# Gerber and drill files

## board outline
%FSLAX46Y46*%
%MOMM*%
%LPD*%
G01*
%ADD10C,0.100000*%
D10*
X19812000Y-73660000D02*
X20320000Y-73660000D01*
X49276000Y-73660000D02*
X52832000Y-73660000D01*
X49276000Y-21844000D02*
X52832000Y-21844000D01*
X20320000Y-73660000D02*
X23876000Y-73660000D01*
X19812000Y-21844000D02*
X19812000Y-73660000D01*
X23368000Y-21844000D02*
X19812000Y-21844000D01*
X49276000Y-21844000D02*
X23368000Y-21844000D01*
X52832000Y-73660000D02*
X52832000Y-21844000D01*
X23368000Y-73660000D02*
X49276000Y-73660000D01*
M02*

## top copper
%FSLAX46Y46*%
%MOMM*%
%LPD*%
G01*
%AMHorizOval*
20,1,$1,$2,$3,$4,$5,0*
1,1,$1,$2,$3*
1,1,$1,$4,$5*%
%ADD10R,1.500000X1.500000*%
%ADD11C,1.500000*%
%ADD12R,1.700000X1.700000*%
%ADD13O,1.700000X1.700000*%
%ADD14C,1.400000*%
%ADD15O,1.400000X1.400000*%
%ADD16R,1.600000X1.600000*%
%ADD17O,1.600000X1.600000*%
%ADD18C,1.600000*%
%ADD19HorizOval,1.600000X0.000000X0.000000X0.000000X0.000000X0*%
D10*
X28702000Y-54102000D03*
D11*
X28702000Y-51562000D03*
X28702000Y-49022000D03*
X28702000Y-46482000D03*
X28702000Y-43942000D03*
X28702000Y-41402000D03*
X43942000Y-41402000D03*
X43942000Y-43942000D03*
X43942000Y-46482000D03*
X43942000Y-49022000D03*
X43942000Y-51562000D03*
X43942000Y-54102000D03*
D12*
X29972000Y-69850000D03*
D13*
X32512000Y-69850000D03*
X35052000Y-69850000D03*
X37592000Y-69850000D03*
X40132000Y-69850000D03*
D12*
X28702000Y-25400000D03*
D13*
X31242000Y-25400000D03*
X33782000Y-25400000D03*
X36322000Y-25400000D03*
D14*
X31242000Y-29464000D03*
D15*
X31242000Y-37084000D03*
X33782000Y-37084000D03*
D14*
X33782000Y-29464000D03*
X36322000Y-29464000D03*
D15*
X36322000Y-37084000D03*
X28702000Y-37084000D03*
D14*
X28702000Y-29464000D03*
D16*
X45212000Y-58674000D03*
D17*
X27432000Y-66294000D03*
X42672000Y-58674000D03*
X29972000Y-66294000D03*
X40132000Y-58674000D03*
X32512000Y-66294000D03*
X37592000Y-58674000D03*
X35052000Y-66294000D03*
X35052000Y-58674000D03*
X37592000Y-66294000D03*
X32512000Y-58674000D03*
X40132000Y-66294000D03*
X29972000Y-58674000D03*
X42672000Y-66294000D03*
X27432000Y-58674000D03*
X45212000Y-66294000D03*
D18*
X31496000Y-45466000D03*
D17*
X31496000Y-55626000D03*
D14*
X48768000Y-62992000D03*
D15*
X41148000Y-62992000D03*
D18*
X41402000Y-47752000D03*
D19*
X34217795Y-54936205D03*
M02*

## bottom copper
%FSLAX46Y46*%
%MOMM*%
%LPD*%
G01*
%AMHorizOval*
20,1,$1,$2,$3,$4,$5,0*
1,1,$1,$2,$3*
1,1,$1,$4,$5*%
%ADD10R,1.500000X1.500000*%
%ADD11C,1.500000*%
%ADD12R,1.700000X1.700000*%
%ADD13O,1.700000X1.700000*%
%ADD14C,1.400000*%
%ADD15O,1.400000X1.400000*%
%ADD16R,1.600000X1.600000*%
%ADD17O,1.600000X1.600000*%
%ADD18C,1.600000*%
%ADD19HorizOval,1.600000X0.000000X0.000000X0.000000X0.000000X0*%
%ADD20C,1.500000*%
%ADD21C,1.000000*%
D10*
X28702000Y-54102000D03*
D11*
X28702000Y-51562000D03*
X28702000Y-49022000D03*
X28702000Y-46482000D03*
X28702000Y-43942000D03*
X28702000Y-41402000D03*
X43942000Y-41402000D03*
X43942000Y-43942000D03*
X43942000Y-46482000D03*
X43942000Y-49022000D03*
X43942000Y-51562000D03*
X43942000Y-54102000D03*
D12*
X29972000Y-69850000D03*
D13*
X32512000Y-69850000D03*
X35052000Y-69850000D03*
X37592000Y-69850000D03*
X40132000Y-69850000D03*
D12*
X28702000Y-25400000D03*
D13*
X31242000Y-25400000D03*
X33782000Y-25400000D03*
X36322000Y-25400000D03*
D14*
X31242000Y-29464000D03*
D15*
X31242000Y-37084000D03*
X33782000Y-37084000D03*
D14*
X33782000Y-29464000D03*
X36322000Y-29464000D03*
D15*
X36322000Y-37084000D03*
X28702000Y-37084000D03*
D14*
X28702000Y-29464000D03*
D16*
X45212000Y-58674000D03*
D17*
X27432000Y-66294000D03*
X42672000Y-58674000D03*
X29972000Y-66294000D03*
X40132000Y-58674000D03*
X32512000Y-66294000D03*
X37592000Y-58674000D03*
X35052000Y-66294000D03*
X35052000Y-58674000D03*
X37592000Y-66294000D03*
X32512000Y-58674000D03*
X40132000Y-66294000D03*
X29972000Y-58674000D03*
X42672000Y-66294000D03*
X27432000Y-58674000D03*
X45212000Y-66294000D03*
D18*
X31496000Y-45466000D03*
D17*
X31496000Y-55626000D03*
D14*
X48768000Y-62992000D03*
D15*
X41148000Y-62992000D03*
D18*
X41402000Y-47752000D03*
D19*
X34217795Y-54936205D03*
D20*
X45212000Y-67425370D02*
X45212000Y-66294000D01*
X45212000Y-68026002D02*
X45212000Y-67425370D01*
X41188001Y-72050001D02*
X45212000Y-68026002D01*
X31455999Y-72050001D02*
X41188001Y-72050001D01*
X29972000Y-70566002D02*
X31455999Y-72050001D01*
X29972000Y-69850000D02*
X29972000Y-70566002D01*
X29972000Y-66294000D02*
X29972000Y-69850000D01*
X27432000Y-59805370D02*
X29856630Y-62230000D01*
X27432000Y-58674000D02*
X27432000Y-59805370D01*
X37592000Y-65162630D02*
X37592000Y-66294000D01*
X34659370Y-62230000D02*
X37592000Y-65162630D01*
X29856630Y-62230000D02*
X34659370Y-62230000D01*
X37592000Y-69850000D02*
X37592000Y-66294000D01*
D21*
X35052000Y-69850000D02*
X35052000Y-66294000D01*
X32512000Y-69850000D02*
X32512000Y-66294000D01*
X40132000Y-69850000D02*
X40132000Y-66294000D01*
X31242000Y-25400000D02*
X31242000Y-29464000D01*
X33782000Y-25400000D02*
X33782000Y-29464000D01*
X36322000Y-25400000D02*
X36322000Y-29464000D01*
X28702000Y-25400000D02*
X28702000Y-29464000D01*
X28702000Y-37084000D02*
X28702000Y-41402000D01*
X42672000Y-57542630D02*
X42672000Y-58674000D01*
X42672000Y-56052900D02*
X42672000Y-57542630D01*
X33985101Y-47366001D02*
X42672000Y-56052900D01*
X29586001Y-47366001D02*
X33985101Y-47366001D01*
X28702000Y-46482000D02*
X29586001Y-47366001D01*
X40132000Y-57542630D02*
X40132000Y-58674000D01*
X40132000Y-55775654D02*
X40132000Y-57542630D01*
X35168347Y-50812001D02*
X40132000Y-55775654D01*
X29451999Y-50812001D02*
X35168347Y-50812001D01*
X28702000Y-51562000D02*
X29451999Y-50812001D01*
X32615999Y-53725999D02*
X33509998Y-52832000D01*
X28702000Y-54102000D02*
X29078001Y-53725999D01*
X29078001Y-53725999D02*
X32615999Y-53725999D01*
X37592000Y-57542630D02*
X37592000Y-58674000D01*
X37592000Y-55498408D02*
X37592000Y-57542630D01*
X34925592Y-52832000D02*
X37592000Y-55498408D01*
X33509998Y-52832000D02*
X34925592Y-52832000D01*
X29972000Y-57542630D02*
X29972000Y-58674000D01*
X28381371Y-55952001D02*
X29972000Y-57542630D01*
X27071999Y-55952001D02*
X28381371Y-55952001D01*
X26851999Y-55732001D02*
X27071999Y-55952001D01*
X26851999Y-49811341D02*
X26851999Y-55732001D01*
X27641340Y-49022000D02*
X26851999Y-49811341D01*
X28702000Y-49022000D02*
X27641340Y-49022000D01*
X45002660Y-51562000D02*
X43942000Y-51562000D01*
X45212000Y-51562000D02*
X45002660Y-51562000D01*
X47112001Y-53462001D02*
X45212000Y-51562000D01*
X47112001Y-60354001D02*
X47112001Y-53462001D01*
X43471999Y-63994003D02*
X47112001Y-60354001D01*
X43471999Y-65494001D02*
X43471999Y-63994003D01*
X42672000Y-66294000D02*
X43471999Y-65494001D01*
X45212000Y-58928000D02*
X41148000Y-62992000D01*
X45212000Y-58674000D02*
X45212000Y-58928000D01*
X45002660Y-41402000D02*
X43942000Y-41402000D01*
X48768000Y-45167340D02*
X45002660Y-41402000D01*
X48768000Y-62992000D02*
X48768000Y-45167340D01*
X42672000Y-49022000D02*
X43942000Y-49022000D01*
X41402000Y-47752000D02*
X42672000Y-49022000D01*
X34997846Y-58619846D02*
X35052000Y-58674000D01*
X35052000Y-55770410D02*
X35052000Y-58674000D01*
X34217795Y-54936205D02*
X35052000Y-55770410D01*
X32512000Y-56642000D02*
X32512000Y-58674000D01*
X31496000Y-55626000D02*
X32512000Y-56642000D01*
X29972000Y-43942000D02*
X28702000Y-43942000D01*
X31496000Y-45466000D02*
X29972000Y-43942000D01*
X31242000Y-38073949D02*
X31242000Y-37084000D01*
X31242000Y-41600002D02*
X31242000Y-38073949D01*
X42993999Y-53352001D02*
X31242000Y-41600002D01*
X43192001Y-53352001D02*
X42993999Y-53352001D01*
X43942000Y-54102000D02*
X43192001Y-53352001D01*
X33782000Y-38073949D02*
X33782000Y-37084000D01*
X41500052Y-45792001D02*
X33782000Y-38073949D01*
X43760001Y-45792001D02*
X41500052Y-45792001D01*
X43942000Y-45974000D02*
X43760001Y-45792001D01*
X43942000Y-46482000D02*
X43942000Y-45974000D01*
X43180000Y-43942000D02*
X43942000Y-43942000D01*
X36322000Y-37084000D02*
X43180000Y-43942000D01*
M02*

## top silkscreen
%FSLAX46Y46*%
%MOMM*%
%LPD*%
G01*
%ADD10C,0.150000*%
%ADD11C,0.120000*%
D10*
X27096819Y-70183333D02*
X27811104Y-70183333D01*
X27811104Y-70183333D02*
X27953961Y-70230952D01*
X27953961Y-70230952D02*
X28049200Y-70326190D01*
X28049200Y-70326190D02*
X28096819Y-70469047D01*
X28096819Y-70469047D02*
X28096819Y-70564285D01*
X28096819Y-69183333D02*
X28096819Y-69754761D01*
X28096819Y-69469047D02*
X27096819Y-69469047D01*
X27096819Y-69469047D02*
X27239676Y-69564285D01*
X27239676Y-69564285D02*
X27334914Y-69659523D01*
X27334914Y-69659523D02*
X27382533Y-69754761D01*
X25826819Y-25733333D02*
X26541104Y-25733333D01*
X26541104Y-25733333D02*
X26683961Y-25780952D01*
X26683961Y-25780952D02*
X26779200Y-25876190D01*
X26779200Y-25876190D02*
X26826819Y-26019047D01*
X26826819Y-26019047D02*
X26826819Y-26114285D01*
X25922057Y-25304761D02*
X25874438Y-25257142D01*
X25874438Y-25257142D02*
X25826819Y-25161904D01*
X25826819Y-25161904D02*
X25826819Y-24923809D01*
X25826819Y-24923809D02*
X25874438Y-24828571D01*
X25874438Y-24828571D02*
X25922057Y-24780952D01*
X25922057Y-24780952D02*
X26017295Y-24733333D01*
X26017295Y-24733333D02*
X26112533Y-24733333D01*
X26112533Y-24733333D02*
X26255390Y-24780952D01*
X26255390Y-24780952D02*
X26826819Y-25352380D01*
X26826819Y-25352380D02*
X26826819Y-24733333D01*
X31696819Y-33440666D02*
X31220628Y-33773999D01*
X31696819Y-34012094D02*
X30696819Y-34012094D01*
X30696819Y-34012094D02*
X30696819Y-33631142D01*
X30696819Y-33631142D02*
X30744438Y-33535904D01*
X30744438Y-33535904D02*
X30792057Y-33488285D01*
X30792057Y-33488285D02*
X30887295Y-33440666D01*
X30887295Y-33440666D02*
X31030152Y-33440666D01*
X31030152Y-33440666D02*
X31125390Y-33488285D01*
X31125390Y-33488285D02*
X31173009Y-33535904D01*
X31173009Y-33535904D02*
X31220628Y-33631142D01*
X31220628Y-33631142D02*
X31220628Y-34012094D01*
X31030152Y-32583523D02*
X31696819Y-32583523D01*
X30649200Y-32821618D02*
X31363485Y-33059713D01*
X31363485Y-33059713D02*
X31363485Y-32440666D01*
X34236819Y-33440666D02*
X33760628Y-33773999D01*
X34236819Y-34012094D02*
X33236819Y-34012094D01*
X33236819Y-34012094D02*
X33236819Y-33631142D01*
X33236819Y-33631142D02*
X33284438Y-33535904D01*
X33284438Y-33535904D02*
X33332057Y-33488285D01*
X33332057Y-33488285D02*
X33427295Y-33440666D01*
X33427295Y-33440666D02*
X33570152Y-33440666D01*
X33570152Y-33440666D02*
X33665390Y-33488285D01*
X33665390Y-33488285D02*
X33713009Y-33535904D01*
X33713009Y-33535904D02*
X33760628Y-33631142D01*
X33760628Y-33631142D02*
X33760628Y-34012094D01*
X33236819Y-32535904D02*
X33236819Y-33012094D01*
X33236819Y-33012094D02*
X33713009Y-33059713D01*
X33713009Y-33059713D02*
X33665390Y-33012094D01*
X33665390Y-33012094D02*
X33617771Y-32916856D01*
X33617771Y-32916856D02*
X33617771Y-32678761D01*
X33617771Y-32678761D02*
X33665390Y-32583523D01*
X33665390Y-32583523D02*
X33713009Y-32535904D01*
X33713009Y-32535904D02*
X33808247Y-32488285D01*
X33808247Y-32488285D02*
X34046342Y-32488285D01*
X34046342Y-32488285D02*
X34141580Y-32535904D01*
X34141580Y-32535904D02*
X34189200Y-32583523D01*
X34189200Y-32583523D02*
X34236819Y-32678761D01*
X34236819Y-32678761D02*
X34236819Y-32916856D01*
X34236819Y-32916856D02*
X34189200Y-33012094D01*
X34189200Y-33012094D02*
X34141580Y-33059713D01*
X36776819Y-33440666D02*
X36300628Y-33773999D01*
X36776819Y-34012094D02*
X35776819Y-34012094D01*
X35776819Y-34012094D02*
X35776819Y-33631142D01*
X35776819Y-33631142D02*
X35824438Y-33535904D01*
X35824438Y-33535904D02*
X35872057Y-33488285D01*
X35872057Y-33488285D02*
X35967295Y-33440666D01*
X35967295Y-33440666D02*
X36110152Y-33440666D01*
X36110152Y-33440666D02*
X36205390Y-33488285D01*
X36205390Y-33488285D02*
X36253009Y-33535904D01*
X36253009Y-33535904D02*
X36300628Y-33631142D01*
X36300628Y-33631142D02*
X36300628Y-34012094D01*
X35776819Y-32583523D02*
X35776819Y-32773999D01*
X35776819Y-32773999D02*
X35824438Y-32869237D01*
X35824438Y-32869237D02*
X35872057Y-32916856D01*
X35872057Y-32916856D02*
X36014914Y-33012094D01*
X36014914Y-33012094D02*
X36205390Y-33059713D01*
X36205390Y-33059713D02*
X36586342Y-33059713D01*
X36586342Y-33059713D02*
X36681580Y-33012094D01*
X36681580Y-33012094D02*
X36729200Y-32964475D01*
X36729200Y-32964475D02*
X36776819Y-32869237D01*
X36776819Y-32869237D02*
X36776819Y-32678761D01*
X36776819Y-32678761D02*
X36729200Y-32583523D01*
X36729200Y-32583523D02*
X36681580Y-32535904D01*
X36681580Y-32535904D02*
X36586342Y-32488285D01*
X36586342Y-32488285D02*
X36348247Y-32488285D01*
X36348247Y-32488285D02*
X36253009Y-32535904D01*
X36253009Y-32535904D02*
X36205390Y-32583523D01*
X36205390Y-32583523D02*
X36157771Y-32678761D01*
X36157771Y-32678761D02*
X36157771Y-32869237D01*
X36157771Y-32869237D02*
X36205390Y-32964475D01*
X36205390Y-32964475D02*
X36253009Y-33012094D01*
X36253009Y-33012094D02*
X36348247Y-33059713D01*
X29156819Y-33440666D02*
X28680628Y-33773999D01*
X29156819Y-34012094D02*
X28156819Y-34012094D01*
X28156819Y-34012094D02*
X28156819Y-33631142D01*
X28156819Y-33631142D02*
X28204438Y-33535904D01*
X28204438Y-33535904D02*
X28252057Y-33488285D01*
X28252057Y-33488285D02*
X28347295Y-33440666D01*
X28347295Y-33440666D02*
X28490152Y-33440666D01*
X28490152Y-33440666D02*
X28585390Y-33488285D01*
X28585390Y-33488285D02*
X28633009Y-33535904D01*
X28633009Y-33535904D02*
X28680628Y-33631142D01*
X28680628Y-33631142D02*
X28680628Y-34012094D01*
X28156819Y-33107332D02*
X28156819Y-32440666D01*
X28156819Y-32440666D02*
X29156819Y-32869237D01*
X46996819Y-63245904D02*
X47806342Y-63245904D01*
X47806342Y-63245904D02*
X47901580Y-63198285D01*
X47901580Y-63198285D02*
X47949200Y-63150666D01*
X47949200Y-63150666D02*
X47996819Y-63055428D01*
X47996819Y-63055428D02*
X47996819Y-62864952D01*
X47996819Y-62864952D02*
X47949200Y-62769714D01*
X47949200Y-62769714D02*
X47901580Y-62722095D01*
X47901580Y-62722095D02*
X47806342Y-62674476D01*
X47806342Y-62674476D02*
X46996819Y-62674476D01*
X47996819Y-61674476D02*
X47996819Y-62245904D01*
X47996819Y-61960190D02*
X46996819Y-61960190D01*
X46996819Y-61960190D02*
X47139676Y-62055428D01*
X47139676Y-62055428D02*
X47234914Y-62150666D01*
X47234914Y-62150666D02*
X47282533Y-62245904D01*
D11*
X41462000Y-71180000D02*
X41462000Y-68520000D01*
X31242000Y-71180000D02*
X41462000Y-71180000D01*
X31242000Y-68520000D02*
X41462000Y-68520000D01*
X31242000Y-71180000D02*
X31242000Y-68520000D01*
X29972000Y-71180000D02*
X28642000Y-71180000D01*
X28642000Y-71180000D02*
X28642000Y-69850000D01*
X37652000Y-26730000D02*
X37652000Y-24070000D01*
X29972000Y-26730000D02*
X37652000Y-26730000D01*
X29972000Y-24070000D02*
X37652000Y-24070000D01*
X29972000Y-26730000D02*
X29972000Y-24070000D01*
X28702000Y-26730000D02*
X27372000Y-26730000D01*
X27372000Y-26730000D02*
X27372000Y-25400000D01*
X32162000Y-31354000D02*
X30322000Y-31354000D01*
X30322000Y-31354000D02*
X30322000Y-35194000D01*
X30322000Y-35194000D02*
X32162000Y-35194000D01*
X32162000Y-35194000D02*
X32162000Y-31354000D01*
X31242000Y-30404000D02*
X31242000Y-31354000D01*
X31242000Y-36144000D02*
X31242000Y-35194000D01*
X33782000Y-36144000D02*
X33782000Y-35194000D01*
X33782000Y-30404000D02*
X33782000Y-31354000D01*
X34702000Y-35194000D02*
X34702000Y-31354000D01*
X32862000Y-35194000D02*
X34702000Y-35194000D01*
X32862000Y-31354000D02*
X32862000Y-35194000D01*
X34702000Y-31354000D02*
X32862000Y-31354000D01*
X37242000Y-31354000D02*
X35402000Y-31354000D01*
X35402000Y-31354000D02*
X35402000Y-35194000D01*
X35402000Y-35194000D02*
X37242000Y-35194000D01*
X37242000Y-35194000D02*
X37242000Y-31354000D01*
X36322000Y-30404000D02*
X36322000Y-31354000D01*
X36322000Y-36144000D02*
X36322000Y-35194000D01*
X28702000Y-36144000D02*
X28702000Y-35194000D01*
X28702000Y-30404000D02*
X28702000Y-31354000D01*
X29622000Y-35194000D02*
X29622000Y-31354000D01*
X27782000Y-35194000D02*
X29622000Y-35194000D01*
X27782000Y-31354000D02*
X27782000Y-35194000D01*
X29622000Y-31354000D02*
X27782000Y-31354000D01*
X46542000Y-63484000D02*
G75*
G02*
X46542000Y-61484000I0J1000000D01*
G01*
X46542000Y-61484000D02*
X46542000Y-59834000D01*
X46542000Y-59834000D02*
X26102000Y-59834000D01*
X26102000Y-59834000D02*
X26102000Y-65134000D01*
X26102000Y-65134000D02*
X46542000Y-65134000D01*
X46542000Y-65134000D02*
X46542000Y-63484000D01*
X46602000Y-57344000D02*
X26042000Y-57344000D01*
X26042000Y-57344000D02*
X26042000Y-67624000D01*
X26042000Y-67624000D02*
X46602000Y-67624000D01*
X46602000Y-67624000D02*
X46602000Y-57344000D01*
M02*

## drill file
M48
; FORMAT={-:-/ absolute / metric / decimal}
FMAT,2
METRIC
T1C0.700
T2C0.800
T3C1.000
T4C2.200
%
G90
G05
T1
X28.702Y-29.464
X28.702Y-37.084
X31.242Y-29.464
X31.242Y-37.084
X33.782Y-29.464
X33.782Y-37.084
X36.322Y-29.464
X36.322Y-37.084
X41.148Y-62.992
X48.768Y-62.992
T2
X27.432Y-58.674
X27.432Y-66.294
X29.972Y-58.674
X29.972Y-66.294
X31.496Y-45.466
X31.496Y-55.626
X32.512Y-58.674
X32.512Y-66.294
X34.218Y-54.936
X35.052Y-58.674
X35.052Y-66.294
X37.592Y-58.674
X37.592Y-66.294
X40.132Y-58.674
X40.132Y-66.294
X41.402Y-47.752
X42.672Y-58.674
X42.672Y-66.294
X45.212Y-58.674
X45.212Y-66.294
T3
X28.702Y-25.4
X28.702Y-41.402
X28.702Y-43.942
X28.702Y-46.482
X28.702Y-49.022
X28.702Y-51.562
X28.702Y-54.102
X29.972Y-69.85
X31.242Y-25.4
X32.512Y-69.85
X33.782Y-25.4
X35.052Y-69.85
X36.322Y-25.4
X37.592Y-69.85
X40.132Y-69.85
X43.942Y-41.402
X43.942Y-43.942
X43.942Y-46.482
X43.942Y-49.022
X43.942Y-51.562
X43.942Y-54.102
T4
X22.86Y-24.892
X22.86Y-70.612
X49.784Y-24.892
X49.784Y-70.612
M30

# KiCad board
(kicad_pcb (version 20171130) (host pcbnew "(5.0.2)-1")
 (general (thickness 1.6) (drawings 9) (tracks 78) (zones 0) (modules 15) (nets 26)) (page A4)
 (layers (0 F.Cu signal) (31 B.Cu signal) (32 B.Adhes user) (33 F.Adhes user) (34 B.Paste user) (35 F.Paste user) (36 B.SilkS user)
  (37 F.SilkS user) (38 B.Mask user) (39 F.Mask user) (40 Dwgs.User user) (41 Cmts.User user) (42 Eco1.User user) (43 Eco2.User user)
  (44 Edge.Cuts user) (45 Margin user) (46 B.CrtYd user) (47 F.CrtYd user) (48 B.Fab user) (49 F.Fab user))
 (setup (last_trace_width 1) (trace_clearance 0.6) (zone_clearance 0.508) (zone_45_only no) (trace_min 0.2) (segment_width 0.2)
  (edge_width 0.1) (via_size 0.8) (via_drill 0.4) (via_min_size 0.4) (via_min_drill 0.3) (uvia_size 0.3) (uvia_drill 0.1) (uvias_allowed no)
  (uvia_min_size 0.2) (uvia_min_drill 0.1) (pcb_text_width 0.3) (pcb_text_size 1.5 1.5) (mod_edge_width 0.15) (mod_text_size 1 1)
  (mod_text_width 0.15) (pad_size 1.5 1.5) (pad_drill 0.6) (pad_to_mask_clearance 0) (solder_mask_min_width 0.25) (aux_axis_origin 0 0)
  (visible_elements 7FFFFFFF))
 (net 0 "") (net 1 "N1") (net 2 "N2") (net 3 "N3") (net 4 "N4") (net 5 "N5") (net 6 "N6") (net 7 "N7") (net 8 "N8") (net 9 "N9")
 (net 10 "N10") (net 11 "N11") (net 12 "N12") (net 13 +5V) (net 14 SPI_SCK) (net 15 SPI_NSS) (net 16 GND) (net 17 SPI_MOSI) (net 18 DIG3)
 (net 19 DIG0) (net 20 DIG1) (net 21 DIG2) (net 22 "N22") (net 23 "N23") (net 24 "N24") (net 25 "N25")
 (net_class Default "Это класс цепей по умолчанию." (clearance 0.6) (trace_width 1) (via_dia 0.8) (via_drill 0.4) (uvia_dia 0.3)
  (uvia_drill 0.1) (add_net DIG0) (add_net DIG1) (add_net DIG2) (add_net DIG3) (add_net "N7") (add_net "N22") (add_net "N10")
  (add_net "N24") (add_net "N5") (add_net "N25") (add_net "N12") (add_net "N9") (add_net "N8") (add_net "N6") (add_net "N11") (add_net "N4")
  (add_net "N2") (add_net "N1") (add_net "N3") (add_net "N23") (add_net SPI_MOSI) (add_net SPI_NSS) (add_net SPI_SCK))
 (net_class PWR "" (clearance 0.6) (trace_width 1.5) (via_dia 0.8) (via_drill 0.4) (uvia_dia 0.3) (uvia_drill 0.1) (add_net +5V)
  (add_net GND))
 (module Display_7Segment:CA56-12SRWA (layer B.Cu) (at 28.702 54.102)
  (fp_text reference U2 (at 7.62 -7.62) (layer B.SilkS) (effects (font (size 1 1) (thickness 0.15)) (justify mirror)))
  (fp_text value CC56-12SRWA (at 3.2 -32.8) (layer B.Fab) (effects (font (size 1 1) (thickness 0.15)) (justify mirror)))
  (pad 1 thru_hole rect (at 0 0) (size 1.5 1.5) (drill 1) (layers *.Cu *.Mask) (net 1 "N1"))
  (pad 2 thru_hole circle (at 0 -2.54) (size 1.5 1.5) (drill 1) (layers *.Cu *.Mask) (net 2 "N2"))
  (pad 3 thru_hole circle (at 0 -5.08) (size 1.5 1.5) (drill 1) (layers *.Cu *.Mask) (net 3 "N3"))
  (pad 4 thru_hole circle (at 0 -7.62) (size 1.5 1.5) (drill 1) (layers *.Cu *.Mask) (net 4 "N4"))
  (pad 5 thru_hole circle (at 0 -10.16) (size 1.5 1.5) (drill 1) (layers *.Cu *.Mask) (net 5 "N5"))
  (pad 6 thru_hole circle (at 0 -12.7) (size 1.5 1.5) (drill 1) (layers *.Cu *.Mask) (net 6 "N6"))
  (pad 7 thru_hole circle (at 15.24 -12.7) (size 1.5 1.5) (drill 1) (layers *.Cu *.Mask) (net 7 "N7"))
  (pad 8 thru_hole circle (at 15.24 -10.16) (size 1.5 1.5) (drill 1) (layers *.Cu *.Mask) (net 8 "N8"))
  (pad 9 thru_hole circle (at 15.24 -7.62) (size 1.5 1.5) (drill 1) (layers *.Cu *.Mask) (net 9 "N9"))
  (pad 10 thru_hole circle (at 15.24 -5.08) (size 1.5 1.5) (drill 1) (layers *.Cu *.Mask) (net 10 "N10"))
  (pad 11 thru_hole circle (at 15.24 -2.54) (size 1.5 1.5) (drill 1) (layers *.Cu *.Mask) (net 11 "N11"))
  (pad 12 thru_hole circle (at 15.24 0) (size 1.5 1.5) (drill 1) (layers *.Cu *.Mask) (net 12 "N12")))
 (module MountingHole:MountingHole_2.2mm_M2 (layer F.Cu) (at 22.86 24.892)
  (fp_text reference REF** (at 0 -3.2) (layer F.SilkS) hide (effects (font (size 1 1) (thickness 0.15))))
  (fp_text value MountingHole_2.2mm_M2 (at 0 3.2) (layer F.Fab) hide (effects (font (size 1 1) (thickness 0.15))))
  (pad 1 np_thru_hole circle (at 0 0) (size 2.2 2.2) (drill 2.2) (layers *.Cu *.Mask)))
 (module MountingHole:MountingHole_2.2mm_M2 (layer F.Cu) (at 22.86 70.612)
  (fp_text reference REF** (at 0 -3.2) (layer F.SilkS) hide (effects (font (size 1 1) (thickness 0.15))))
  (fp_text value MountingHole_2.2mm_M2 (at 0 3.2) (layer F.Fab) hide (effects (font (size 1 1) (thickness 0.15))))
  (pad 1 np_thru_hole circle (at 0 0) (size 2.2 2.2) (drill 2.2) (layers *.Cu *.Mask)))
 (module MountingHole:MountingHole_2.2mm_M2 (layer F.Cu) (at 49.784 24.892)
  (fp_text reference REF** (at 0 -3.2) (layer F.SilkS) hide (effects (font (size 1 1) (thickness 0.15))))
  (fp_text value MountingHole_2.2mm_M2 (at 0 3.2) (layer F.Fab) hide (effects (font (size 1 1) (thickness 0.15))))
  (pad 1 np_thru_hole circle (at 0 0) (size 2.2 2.2) (drill 2.2) (layers *.Cu *.Mask)))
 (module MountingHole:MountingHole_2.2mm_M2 (layer F.Cu) (at 49.784 70.612)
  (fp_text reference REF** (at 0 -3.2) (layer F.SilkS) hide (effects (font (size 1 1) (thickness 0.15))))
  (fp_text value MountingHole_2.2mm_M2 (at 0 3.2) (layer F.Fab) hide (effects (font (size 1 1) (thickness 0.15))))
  (pad 1 np_thru_hole circle (at 0 0) (size 2.2 2.2) (drill 2.2) (layers *.Cu *.Mask)))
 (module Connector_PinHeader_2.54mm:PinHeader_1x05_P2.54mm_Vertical (layer F.Cu) (at 29.972 69.85 90)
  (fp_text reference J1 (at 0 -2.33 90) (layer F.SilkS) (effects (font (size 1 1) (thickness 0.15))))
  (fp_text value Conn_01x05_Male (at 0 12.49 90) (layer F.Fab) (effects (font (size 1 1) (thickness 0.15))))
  (fp_line (start -1.33 11.49) (end 1.33 11.49) (layer F.SilkS) (width 0.12))
  (fp_line (start -1.33 1.27) (end -1.33 11.49) (layer F.SilkS) (width 0.12))
  (fp_line (start 1.33 1.27) (end 1.33 11.49) (layer F.SilkS) (width 0.12))
  (fp_line (start -1.33 1.27) (end 1.33 1.27) (layer F.SilkS) (width 0.12))
  (fp_line (start -1.33 0) (end -1.33 -1.33) (layer F.SilkS) (width 0.12))
  (fp_line (start -1.33 -1.33) (end 0 -1.33) (layer F.SilkS) (width 0.12))
  (pad 1 thru_hole rect (at 0 0 90) (size 1.7 1.7) (drill 1) (layers *.Cu *.Mask) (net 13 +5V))
  (pad 2 thru_hole oval (at 0 2.54 90) (size 1.7 1.7) (drill 1) (layers *.Cu *.Mask) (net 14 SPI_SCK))
  (pad 3 thru_hole oval (at 0 5.08 90) (size 1.7 1.7) (drill 1) (layers *.Cu *.Mask) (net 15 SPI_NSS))
  (pad 4 thru_hole oval (at 0 7.62 90) (size 1.7 1.7) (drill 1) (layers *.Cu *.Mask) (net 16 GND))
  (pad 5 thru_hole oval (at 0 10.16 90) (size 1.7 1.7) (drill 1) (layers *.Cu *.Mask) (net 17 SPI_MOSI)))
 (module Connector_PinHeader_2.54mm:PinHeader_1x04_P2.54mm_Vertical (layer F.Cu) (at 28.702 25.4 90)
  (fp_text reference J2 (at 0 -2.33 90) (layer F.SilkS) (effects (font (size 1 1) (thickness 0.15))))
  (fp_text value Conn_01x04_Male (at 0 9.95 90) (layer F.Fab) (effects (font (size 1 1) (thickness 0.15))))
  (fp_line (start -1.33 8.95) (end 1.33 8.95) (layer F.SilkS) (width 0.12))
  (fp_line (start -1.33 1.27) (end -1.33 8.95) (layer F.SilkS) (width 0.12))
  (fp_line (start 1.33 1.27) (end 1.33 8.95) (layer F.SilkS) (width 0.12))
  (fp_line (start -1.33 1.27) (end 1.33 1.27) (layer F.SilkS) (width 0.12))
  (fp_line (start -1.33 0) (end -1.33 -1.33) (layer F.SilkS) (width 0.12))
  (fp_line (start -1.33 -1.33) (end 0 -1.33) (layer F.SilkS) (width 0.12))
  (pad 1 thru_hole rect (at 0 0 90) (size 1.7 1.7) (drill 1) (layers *.Cu *.Mask) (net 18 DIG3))
  (pad 2 thru_hole oval (at 0 2.54 90) (size 1.7 1.7) (drill 1) (layers *.Cu *.Mask) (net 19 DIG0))
  (pad 3 thru_hole oval (at 0 5.08 90) (size 1.7 1.7) (drill 1) (layers *.Cu *.Mask) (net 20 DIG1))
  (pad 4 thru_hole oval (at 0 7.62 90) (size 1.7 1.7) (drill 1) (layers *.Cu *.Mask) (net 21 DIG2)))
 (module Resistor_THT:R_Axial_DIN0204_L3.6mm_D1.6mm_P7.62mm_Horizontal (layer F.Cu) (at 31.242 29.464 270)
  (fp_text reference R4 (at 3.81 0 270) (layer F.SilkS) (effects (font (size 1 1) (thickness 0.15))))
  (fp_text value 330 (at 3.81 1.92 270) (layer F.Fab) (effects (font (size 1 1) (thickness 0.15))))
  (fp_line (start 1.89 -0.92) (end 1.89 0.92) (layer F.SilkS) (width 0.12))
  (fp_line (start 1.89 0.92) (end 5.73 0.92) (layer F.SilkS) (width 0.12))
  (fp_line (start 5.73 0.92) (end 5.73 -0.92) (layer F.SilkS) (width 0.12))
  (fp_line (start 5.73 -0.92) (end 1.89 -0.92) (layer F.SilkS) (width 0.12))
  (fp_line (start 0.94 0) (end 1.89 0) (layer F.SilkS) (width 0.12))
  (fp_line (start 6.68 0) (end 5.73 0) (layer F.SilkS) (width 0.12))
  (pad 1 thru_hole circle (at 0 0 270) (size 1.4 1.4) (drill 0.7) (layers *.Cu *.Mask) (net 19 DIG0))
  (pad 2 thru_hole oval (at 7.62 0 270) (size 1.4 1.4) (drill 0.7) (layers *.Cu *.Mask) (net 12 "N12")))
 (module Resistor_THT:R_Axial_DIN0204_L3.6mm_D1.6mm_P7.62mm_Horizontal (layer F.Cu) (at 33.782 29.464 270)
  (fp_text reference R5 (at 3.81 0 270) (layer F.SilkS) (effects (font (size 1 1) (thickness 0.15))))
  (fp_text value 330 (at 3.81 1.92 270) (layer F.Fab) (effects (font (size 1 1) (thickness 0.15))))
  (fp_line (start 6.68 0) (end 5.73 0) (layer F.SilkS) (width 0.12))
  (fp_line (start 0.94 0) (end 1.89 0) (layer F.SilkS) (width 0.12))
  (fp_line (start 5.73 -0.92) (end 1.89 -0.92) (layer F.SilkS) (width 0.12))
  (fp_line (start 5.73 0.92) (end 5.73 -0.92) (layer F.SilkS) (width 0.12))
  (fp_line (start 1.89 0.92) (end 5.73 0.92) (layer F.SilkS) (width 0.12))
  (fp_line (start 1.89 -0.92) (end 1.89 0.92) (layer F.SilkS) (width 0.12))
  (pad 2 thru_hole oval (at 7.62 0 270) (size 1.4 1.4) (drill 0.7) (layers *.Cu *.Mask) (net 9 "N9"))
  (pad 1 thru_hole circle (at 0 0 270) (size 1.4 1.4) (drill 0.7) (layers *.Cu *.Mask) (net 20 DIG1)))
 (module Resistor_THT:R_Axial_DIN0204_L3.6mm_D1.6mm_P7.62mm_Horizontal (layer F.Cu) (at 36.322 29.464 270)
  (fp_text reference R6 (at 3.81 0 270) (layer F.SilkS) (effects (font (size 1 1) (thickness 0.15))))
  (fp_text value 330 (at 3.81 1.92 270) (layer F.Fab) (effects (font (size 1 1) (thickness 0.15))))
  (fp_line (start 1.89 -0.92) (end 1.89 0.92) (layer F.SilkS) (width 0.12))
  (fp_line (start 1.89 0.92) (end 5.73 0.92) (layer F.SilkS) (width 0.12))
  (fp_line (start 5.73 0.92) (end 5.73 -0.92) (layer F.SilkS) (width 0.12))
  (fp_line (start 5.73 -0.92) (end 1.89 -0.92) (layer F.SilkS) (width 0.12))
  (fp_line (start 0.94 0) (end 1.89 0) (layer F.SilkS) (width 0.12))
  (fp_line (start 6.68 0) (end 5.73 0) (layer F.SilkS) (width 0.12))
  (pad 1 thru_hole circle (at 0 0 270) (size 1.4 1.4) (drill 0.7) (layers *.Cu *.Mask) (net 21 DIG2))
  (pad 2 thru_hole oval (at 7.62 0 270) (size 1.4 1.4) (drill 0.7) (layers *.Cu *.Mask) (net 8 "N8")))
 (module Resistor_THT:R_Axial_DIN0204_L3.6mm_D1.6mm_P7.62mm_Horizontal (layer F.Cu) (at 28.702 29.464 270)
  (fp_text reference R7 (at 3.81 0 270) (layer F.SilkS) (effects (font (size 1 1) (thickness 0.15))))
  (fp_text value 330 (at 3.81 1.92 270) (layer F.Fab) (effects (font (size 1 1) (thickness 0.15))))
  (fp_line (start 6.68 0) (end 5.73 0) (layer F.SilkS) (width 0.12))
  (fp_line (start 0.94 0) (end 1.89 0) (layer F.SilkS) (width 0.12))
  (fp_line (start 5.73 -0.92) (end 1.89 -0.92) (layer F.SilkS) (width 0.12))
  (fp_line (start 5.73 0.92) (end 5.73 -0.92) (layer F.SilkS) (width 0.12))
  (fp_line (start 1.89 0.92) (end 5.73 0.92) (layer F.SilkS) (width 0.12))
  (fp_line (start 1.89 -0.92) (end 1.89 0.92) (layer F.SilkS) (width 0.12))
  (pad 2 thru_hole oval (at 7.62 0 270) (size 1.4 1.4) (drill 0.7) (layers *.Cu *.Mask) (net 6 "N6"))
  (pad 1 thru_hole circle (at 0 0 270) (size 1.4 1.4) (drill 0.7) (layers *.Cu *.Mask) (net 18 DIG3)))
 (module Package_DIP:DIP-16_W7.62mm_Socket (layer F.Cu) (at 45.212 58.674 270)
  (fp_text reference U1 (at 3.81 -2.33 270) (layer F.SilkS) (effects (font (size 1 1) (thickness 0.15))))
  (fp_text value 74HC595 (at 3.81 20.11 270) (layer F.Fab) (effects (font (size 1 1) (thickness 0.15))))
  (fp_arc (start 3.81 -1.33) (end 2.81 -1.33) (angle -180) (layer F.SilkS) (width 0.12))
  (fp_line (start 2.81 -1.33) (end 1.16 -1.33) (layer F.SilkS) (width 0.12))
  (fp_line (start 1.16 -1.33) (end 1.16 19.11) (layer F.SilkS) (width 0.12))
  (fp_line (start 1.16 19.11) (end 6.46 19.11) (layer F.SilkS) (width 0.12))
  (fp_line (start 6.46 19.11) (end 6.46 -1.33) (layer F.SilkS) (width 0.12))
  (fp_line (start 6.46 -1.33) (end 4.81 -1.33) (layer F.SilkS) (width 0.12))
  (fp_line (start -1.33 -1.39) (end -1.33 19.17) (layer F.SilkS) (width 0.12))
  (fp_line (start -1.33 19.17) (end 8.95 19.17) (layer F.SilkS) (width 0.12))
  (fp_line (start 8.95 19.17) (end 8.95 -1.39) (layer F.SilkS) (width 0.12))
  (fp_line (start 8.95 -1.39) (end -1.33 -1.39) (layer F.SilkS) (width 0.12))
  (pad 1 thru_hole rect (at 0 0 270) (size 1.6 1.6) (drill 0.8) (layers *.Cu *.Mask) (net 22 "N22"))
  (pad 9 thru_hole oval (at 7.62 17.78 270) (size 1.6 1.6) (drill 0.8) (layers *.Cu *.Mask) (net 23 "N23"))
  (pad 2 thru_hole oval (at 0 2.54 270) (size 1.6 1.6) (drill 0.8) (layers *.Cu *.Mask) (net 4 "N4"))
  (pad 10 thru_hole oval (at 7.62 15.24 270) (size 1.6 1.6) (drill 0.8) (layers *.Cu *.Mask) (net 13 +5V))
  (pad 3 thru_hole oval (at 0 5.08 270) (size 1.6 1.6) (drill 0.8) (layers *.Cu *.Mask) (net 2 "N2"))
  (pad 11 thru_hole oval (at 7.62 12.7 270) (size 1.6 1.6) (drill 0.8) (layers *.Cu *.Mask) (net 14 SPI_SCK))
  (pad 4 thru_hole oval (at 0 7.62 270) (size 1.6 1.6) (drill 0.8) (layers *.Cu *.Mask) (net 1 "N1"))
  (pad 12 thru_hole oval (at 7.62 10.16 270) (size 1.6 1.6) (drill 0.8) (layers *.Cu *.Mask) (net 15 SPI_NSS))
  (pad 5 thru_hole oval (at 0 10.16 270) (size 1.6 1.6) (drill 0.8) (layers *.Cu *.Mask) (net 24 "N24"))
  (pad 13 thru_hole oval (at 7.62 7.62 270) (size 1.6 1.6) (drill 0.8) (layers *.Cu *.Mask) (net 16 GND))
  (pad 6 thru_hole oval (at 0 12.7 270) (size 1.6 1.6) (drill 0.8) (layers *.Cu *.Mask) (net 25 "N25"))
  (pad 14 thru_hole oval (at 7.62 5.08 270) (size 1.6 1.6) (drill 0.8) (layers *.Cu *.Mask) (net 17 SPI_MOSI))
  (pad 7 thru_hole oval (at 0 15.24 270) (size 1.6 1.6) (drill 0.8) (layers *.Cu *.Mask) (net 3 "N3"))
  (pad 15 thru_hole oval (at 7.62 2.54 270) (size 1.6 1.6) (drill 0.8) (layers *.Cu *.Mask) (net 11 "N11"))
  (pad 8 thru_hole oval (at 0 17.78 270) (size 1.6 1.6) (drill 0.8) (layers *.Cu *.Mask) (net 16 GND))
  (pad 16 thru_hole oval (at 7.62 0 270) (size 1.6 1.6) (drill 0.8) (layers *.Cu *.Mask) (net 13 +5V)))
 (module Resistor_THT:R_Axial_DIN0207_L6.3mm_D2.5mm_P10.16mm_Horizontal (layer B.Cu) (at 31.496 45.466 270)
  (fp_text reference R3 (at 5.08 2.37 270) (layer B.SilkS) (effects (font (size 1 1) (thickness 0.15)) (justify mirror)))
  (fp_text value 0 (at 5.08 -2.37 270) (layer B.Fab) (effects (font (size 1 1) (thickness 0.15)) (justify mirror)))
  (pad 1 thru_hole circle (at 0 0 270) (size 1.6 1.6) (drill 0.8) (layers *.Cu *.Mask) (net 5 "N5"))
  (pad 2 thru_hole oval (at 10.16 0 270) (size 1.6 1.6) (drill 0.8) (layers *.Cu *.Mask) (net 25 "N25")))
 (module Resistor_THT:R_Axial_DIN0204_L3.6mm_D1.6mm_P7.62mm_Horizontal (layer B.Cu) (at 48.768 62.992 180)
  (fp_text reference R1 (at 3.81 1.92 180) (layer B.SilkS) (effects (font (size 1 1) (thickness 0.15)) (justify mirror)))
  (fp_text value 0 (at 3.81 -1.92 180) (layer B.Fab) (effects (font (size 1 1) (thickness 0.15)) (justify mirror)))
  (pad 1 thru_hole circle (at 0 0 180) (size 1.4 1.4) (drill 0.7) (layers *.Cu *.Mask) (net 7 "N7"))
  (pad 2 thru_hole oval (at 7.62 0 180) (size 1.4 1.4) (drill 0.7) (layers *.Cu *.Mask) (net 22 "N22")))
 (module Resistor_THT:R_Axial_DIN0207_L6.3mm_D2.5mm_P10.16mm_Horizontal (layer B.Cu) (at 41.402 47.752 225)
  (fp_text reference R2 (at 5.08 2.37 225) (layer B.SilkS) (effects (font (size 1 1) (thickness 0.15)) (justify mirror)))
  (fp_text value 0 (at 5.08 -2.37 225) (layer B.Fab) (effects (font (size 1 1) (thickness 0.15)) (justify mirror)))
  (pad 1 thru_hole circle (at 0 0 225) (size 1.6 1.6) (drill 0.8) (layers *.Cu *.Mask) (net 10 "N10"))
  (pad 2 thru_hole oval (at 10.16 0 225) (size 1.6 1.6) (drill 0.8) (layers *.Cu *.Mask) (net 24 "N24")))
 (gr_line (start 19.812 73.66) (end 20.32 73.66) (layer Edge.Cuts) (width 0.1))
 (gr_line (start 49.276 73.66) (end 52.832 73.66) (layer Edge.Cuts) (width 0.1))
 (gr_line (start 49.276 21.844) (end 52.832 21.844) (layer Edge.Cuts) (width 0.1))
 (gr_line (start 20.32 73.66) (end 23.876 73.66) (layer Edge.Cuts) (width 0.1))
 (gr_line (start 19.812 21.844) (end 19.812 73.66) (layer Edge.Cuts) (width 0.1))
 (gr_line (start 23.368 21.844) (end 19.812 21.844) (layer Edge.Cuts) (width 0.1))
 (gr_line (start 49.276 21.844) (end 23.368 21.844) (layer Edge.Cuts) (width 0.1))
 (gr_line (start 52.832 73.66) (end 52.832 21.844) (layer Edge.Cuts) (width 0.1))
 (gr_line (start 23.368 73.66) (end 49.276 73.66) (layer Edge.Cuts) (width 0.1))
 (segment (start 45.212 67.42537) (end 45.212 66.294) (width 1.5) (layer B.Cu) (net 13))
 (segment (start 45.212 68.026002) (end 45.212 67.42537) (width 1.5) (layer B.Cu) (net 13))
 (segment (start 41.188001 72.050001) (end 45.212 68.026002) (width 1.5) (layer B.Cu) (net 13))
 (segment (start 31.455999 72.050001) (end 41.188001 72.050001) (width 1.5) (layer B.Cu) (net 13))
 (segment (start 29.972 70.566002) (end 31.455999 72.050001) (width 1.5) (layer B.Cu) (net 13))
 (segment (start 29.972 69.85) (end 29.972 70.566002) (width 1.5) (layer B.Cu) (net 13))
 (segment (start 29.972 66.294) (end 29.972 69.85) (width 1.5) (layer B.Cu) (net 13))
 (segment (start 27.432 59.80537) (end 29.85663 62.23) (width 1.5) (layer B.Cu) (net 16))
 (segment (start 27.432 58.674) (end 27.432 59.80537) (width 1.5) (layer B.Cu) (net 16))
 (segment (start 37.592 65.16263) (end 37.592 66.294) (width 1.5) (layer B.Cu) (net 16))
 (segment (start 34.65937 62.23) (end 37.592 65.16263) (width 1.5) (layer B.Cu) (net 16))
 (segment (start 29.85663 62.23) (end 34.65937 62.23) (width 1.5) (layer B.Cu) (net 16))
 (segment (start 37.592 69.85) (end 37.592 66.294) (width 1.5) (layer B.Cu) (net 16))
 (segment (start 35.052 69.85) (end 35.052 66.294) (width 1) (layer B.Cu) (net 15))
 (segment (start 32.512 69.85) (end 32.512 66.294) (width 1) (layer B.Cu) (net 14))
 (segment (start 40.132 69.85) (end 40.132 66.294) (width 1) (layer B.Cu) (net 17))
 (segment (start 31.242 25.4) (end 31.242 29.464) (width 1) (layer B.Cu) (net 19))
 (segment (start 33.782 25.4) (end 33.782 29.464) (width 1) (layer B.Cu) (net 20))
 (segment (start 36.322 25.4) (end 36.322 29.464) (width 1) (layer B.Cu) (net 21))
 (segment (start 28.702 25.4) (end 28.702 29.464) (width 1) (layer B.Cu) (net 18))
 (segment (start 28.702 37.084) (end 28.702 41.402) (width 1) (layer B.Cu) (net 6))
 (segment (start 42.672 57.54263) (end 42.672 58.674) (width 1) (layer B.Cu) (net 4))
 (segment (start 42.672 56.0529) (end 42.672 57.54263) (width 1) (layer B.Cu) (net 4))
 (segment (start 33.985101 47.366001) (end 42.672 56.0529) (width 1) (layer B.Cu) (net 4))
 (segment (start 29.586001 47.366001) (end 33.985101 47.366001) (width 1) (layer B.Cu) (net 4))
 (segment (start 28.702 46.482) (end 29.586001 47.366001) (width 1) (layer B.Cu) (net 4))
 (segment (start 40.132 57.54263) (end 40.132 58.674) (width 1) (layer B.Cu) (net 2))
 (segment (start 40.132 55.775654) (end 40.132 57.54263) (width 1) (layer B.Cu) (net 2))
 (segment (start 35.168347 50.812001) (end 40.132 55.775654) (width 1) (layer B.Cu) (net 2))
 (segment (start 29.451999 50.812001) (end 35.168347 50.812001) (width 1) (layer B.Cu) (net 2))
 (segment (start 28.702 51.562) (end 29.451999 50.812001) (width 1) (layer B.Cu) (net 2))
 (segment (start 32.615999 53.725999) (end 33.509998 52.832) (width 1) (layer B.Cu) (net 1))
 (segment (start 28.702 54.102) (end 29.078001 53.725999) (width 1) (layer B.Cu) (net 1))
 (segment (start 29.078001 53.725999) (end 32.615999 53.725999) (width 1) (layer B.Cu) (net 1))
 (segment (start 37.592 57.54263) (end 37.592 58.674) (width 1) (layer B.Cu) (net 1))
 (segment (start 37.592 55.498408) (end 37.592 57.54263) (width 1) (layer B.Cu) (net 1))
 (segment (start 34.925592 52.832) (end 37.592 55.498408) (width 1) (layer B.Cu) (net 1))
 (segment (start 33.509998 52.832) (end 34.925592 52.832) (width 1) (layer B.Cu) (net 1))
 (segment (start 29.972 57.54263) (end 29.972 58.674) (width 1) (layer B.Cu) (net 3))
 (segment (start 28.381371 55.952001) (end 29.972 57.54263) (width 1) (layer B.Cu) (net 3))
 (segment (start 27.071999 55.952001) (end 28.381371 55.952001) (width 1) (layer B.Cu) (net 3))
 (segment (start 26.851999 55.732001) (end 27.071999 55.952001) (width 1) (layer B.Cu) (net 3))
 (segment (start 26.851999 49.811341) (end 26.851999 55.732001) (width 1) (layer B.Cu) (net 3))
 (segment (start 27.64134 49.022) (end 26.851999 49.811341) (width 1) (layer B.Cu) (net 3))
 (segment (start 28.702 49.022) (end 27.64134 49.022) (width 1) (layer B.Cu) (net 3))
 (segment (start 45.00266 51.562) (end 43.942 51.562) (width 1) (layer B.Cu) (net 11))
 (segment (start 45.212 51.562) (end 45.00266 51.562) (width 1) (layer B.Cu) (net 11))
 (segment (start 47.112001 53.462001) (end 45.212 51.562) (width 1) (layer B.Cu) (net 11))
 (segment (start 47.112001 60.354001) (end 47.112001 53.462001) (width 1) (layer B.Cu) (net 11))
 (segment (start 43.471999 63.994003) (end 47.112001 60.354001) (width 1) (layer B.Cu) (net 11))
 (segment (start 43.471999 65.494001) (end 43.471999 63.994003) (width 1) (layer B.Cu) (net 11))
 (segment (start 42.672 66.294) (end 43.471999 65.494001) (width 1) (layer B.Cu) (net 11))
 (segment (start 45.212 58.928) (end 41.148 62.992) (width 1) (layer B.Cu) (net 22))
 (segment (start 45.212 58.674) (end 45.212 58.928) (width 1) (layer B.Cu) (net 22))
 (segment (start 45.00266 41.402) (end 43.942 41.402) (width 1) (layer B.Cu) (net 7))
 (segment (start 48.768 45.16734) (end 45.00266 41.402) (width 1) (layer B.Cu) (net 7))
 (segment (start 48.768 62.992) (end 48.768 45.16734) (width 1) (layer B.Cu) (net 7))
 (segment (start 42.672 49.022) (end 43.942 49.022) (width 1) (layer B.Cu) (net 10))
 (segment (start 41.402 47.752) (end 42.672 49.022) (width 1) (layer B.Cu) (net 10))
 (segment (start 34.997846 58.619846) (end 35.052 58.674) (width 1) (layer B.Cu) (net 24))
 (segment (start 35.052 55.77041) (end 35.052 58.674) (width 1) (layer B.Cu) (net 24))
 (segment (start 34.217795 54.936205) (end 35.052 55.77041) (width 1) (layer B.Cu) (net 24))
 (segment (start 32.512 56.642) (end 32.512 58.674) (width 1) (layer B.Cu) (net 25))
 (segment (start 31.496 55.626) (end 32.512 56.642) (width 1) (layer B.Cu) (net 25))
 (segment (start 29.972 43.942) (end 28.702 43.942) (width 1) (layer B.Cu) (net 5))
 (segment (start 31.496 45.466) (end 29.972 43.942) (width 1) (layer B.Cu) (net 5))
 (segment (start 31.242 38.073949) (end 31.242 37.084) (width 1) (layer B.Cu) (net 12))
 (segment (start 31.242 41.600002) (end 31.242 38.073949) (width 1) (layer B.Cu) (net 12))
 (segment (start 42.993999 53.352001) (end 31.242 41.600002) (width 1) (layer B.Cu) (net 12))
 (segment (start 43.192001 53.352001) (end 42.993999 53.352001) (width 1) (layer B.Cu) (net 12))
 (segment (start 43.942 54.102) (end 43.192001 53.352001) (width 1) (layer B.Cu) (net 12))
 (segment (start 33.782 38.073949) (end 33.782 37.084) (width 1) (layer B.Cu) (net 9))
 (segment (start 41.500052 45.792001) (end 33.782 38.073949) (width 1) (layer B.Cu) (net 9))
 (segment (start 43.760001 45.792001) (end 41.500052 45.792001) (width 1) (layer B.Cu) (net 9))
 (segment (start 43.942 45.974) (end 43.760001 45.792001) (width 1) (layer B.Cu) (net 9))
 (segment (start 43.942 46.482) (end 43.942 45.974) (width 1) (layer B.Cu) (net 9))
 (segment (start 43.18 43.942) (end 43.942 43.942) (width 1) (layer B.Cu) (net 8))
 (segment (start 36.322 37.084) (end 43.18 43.942) (width 1) (layer B.Cu) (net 8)))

